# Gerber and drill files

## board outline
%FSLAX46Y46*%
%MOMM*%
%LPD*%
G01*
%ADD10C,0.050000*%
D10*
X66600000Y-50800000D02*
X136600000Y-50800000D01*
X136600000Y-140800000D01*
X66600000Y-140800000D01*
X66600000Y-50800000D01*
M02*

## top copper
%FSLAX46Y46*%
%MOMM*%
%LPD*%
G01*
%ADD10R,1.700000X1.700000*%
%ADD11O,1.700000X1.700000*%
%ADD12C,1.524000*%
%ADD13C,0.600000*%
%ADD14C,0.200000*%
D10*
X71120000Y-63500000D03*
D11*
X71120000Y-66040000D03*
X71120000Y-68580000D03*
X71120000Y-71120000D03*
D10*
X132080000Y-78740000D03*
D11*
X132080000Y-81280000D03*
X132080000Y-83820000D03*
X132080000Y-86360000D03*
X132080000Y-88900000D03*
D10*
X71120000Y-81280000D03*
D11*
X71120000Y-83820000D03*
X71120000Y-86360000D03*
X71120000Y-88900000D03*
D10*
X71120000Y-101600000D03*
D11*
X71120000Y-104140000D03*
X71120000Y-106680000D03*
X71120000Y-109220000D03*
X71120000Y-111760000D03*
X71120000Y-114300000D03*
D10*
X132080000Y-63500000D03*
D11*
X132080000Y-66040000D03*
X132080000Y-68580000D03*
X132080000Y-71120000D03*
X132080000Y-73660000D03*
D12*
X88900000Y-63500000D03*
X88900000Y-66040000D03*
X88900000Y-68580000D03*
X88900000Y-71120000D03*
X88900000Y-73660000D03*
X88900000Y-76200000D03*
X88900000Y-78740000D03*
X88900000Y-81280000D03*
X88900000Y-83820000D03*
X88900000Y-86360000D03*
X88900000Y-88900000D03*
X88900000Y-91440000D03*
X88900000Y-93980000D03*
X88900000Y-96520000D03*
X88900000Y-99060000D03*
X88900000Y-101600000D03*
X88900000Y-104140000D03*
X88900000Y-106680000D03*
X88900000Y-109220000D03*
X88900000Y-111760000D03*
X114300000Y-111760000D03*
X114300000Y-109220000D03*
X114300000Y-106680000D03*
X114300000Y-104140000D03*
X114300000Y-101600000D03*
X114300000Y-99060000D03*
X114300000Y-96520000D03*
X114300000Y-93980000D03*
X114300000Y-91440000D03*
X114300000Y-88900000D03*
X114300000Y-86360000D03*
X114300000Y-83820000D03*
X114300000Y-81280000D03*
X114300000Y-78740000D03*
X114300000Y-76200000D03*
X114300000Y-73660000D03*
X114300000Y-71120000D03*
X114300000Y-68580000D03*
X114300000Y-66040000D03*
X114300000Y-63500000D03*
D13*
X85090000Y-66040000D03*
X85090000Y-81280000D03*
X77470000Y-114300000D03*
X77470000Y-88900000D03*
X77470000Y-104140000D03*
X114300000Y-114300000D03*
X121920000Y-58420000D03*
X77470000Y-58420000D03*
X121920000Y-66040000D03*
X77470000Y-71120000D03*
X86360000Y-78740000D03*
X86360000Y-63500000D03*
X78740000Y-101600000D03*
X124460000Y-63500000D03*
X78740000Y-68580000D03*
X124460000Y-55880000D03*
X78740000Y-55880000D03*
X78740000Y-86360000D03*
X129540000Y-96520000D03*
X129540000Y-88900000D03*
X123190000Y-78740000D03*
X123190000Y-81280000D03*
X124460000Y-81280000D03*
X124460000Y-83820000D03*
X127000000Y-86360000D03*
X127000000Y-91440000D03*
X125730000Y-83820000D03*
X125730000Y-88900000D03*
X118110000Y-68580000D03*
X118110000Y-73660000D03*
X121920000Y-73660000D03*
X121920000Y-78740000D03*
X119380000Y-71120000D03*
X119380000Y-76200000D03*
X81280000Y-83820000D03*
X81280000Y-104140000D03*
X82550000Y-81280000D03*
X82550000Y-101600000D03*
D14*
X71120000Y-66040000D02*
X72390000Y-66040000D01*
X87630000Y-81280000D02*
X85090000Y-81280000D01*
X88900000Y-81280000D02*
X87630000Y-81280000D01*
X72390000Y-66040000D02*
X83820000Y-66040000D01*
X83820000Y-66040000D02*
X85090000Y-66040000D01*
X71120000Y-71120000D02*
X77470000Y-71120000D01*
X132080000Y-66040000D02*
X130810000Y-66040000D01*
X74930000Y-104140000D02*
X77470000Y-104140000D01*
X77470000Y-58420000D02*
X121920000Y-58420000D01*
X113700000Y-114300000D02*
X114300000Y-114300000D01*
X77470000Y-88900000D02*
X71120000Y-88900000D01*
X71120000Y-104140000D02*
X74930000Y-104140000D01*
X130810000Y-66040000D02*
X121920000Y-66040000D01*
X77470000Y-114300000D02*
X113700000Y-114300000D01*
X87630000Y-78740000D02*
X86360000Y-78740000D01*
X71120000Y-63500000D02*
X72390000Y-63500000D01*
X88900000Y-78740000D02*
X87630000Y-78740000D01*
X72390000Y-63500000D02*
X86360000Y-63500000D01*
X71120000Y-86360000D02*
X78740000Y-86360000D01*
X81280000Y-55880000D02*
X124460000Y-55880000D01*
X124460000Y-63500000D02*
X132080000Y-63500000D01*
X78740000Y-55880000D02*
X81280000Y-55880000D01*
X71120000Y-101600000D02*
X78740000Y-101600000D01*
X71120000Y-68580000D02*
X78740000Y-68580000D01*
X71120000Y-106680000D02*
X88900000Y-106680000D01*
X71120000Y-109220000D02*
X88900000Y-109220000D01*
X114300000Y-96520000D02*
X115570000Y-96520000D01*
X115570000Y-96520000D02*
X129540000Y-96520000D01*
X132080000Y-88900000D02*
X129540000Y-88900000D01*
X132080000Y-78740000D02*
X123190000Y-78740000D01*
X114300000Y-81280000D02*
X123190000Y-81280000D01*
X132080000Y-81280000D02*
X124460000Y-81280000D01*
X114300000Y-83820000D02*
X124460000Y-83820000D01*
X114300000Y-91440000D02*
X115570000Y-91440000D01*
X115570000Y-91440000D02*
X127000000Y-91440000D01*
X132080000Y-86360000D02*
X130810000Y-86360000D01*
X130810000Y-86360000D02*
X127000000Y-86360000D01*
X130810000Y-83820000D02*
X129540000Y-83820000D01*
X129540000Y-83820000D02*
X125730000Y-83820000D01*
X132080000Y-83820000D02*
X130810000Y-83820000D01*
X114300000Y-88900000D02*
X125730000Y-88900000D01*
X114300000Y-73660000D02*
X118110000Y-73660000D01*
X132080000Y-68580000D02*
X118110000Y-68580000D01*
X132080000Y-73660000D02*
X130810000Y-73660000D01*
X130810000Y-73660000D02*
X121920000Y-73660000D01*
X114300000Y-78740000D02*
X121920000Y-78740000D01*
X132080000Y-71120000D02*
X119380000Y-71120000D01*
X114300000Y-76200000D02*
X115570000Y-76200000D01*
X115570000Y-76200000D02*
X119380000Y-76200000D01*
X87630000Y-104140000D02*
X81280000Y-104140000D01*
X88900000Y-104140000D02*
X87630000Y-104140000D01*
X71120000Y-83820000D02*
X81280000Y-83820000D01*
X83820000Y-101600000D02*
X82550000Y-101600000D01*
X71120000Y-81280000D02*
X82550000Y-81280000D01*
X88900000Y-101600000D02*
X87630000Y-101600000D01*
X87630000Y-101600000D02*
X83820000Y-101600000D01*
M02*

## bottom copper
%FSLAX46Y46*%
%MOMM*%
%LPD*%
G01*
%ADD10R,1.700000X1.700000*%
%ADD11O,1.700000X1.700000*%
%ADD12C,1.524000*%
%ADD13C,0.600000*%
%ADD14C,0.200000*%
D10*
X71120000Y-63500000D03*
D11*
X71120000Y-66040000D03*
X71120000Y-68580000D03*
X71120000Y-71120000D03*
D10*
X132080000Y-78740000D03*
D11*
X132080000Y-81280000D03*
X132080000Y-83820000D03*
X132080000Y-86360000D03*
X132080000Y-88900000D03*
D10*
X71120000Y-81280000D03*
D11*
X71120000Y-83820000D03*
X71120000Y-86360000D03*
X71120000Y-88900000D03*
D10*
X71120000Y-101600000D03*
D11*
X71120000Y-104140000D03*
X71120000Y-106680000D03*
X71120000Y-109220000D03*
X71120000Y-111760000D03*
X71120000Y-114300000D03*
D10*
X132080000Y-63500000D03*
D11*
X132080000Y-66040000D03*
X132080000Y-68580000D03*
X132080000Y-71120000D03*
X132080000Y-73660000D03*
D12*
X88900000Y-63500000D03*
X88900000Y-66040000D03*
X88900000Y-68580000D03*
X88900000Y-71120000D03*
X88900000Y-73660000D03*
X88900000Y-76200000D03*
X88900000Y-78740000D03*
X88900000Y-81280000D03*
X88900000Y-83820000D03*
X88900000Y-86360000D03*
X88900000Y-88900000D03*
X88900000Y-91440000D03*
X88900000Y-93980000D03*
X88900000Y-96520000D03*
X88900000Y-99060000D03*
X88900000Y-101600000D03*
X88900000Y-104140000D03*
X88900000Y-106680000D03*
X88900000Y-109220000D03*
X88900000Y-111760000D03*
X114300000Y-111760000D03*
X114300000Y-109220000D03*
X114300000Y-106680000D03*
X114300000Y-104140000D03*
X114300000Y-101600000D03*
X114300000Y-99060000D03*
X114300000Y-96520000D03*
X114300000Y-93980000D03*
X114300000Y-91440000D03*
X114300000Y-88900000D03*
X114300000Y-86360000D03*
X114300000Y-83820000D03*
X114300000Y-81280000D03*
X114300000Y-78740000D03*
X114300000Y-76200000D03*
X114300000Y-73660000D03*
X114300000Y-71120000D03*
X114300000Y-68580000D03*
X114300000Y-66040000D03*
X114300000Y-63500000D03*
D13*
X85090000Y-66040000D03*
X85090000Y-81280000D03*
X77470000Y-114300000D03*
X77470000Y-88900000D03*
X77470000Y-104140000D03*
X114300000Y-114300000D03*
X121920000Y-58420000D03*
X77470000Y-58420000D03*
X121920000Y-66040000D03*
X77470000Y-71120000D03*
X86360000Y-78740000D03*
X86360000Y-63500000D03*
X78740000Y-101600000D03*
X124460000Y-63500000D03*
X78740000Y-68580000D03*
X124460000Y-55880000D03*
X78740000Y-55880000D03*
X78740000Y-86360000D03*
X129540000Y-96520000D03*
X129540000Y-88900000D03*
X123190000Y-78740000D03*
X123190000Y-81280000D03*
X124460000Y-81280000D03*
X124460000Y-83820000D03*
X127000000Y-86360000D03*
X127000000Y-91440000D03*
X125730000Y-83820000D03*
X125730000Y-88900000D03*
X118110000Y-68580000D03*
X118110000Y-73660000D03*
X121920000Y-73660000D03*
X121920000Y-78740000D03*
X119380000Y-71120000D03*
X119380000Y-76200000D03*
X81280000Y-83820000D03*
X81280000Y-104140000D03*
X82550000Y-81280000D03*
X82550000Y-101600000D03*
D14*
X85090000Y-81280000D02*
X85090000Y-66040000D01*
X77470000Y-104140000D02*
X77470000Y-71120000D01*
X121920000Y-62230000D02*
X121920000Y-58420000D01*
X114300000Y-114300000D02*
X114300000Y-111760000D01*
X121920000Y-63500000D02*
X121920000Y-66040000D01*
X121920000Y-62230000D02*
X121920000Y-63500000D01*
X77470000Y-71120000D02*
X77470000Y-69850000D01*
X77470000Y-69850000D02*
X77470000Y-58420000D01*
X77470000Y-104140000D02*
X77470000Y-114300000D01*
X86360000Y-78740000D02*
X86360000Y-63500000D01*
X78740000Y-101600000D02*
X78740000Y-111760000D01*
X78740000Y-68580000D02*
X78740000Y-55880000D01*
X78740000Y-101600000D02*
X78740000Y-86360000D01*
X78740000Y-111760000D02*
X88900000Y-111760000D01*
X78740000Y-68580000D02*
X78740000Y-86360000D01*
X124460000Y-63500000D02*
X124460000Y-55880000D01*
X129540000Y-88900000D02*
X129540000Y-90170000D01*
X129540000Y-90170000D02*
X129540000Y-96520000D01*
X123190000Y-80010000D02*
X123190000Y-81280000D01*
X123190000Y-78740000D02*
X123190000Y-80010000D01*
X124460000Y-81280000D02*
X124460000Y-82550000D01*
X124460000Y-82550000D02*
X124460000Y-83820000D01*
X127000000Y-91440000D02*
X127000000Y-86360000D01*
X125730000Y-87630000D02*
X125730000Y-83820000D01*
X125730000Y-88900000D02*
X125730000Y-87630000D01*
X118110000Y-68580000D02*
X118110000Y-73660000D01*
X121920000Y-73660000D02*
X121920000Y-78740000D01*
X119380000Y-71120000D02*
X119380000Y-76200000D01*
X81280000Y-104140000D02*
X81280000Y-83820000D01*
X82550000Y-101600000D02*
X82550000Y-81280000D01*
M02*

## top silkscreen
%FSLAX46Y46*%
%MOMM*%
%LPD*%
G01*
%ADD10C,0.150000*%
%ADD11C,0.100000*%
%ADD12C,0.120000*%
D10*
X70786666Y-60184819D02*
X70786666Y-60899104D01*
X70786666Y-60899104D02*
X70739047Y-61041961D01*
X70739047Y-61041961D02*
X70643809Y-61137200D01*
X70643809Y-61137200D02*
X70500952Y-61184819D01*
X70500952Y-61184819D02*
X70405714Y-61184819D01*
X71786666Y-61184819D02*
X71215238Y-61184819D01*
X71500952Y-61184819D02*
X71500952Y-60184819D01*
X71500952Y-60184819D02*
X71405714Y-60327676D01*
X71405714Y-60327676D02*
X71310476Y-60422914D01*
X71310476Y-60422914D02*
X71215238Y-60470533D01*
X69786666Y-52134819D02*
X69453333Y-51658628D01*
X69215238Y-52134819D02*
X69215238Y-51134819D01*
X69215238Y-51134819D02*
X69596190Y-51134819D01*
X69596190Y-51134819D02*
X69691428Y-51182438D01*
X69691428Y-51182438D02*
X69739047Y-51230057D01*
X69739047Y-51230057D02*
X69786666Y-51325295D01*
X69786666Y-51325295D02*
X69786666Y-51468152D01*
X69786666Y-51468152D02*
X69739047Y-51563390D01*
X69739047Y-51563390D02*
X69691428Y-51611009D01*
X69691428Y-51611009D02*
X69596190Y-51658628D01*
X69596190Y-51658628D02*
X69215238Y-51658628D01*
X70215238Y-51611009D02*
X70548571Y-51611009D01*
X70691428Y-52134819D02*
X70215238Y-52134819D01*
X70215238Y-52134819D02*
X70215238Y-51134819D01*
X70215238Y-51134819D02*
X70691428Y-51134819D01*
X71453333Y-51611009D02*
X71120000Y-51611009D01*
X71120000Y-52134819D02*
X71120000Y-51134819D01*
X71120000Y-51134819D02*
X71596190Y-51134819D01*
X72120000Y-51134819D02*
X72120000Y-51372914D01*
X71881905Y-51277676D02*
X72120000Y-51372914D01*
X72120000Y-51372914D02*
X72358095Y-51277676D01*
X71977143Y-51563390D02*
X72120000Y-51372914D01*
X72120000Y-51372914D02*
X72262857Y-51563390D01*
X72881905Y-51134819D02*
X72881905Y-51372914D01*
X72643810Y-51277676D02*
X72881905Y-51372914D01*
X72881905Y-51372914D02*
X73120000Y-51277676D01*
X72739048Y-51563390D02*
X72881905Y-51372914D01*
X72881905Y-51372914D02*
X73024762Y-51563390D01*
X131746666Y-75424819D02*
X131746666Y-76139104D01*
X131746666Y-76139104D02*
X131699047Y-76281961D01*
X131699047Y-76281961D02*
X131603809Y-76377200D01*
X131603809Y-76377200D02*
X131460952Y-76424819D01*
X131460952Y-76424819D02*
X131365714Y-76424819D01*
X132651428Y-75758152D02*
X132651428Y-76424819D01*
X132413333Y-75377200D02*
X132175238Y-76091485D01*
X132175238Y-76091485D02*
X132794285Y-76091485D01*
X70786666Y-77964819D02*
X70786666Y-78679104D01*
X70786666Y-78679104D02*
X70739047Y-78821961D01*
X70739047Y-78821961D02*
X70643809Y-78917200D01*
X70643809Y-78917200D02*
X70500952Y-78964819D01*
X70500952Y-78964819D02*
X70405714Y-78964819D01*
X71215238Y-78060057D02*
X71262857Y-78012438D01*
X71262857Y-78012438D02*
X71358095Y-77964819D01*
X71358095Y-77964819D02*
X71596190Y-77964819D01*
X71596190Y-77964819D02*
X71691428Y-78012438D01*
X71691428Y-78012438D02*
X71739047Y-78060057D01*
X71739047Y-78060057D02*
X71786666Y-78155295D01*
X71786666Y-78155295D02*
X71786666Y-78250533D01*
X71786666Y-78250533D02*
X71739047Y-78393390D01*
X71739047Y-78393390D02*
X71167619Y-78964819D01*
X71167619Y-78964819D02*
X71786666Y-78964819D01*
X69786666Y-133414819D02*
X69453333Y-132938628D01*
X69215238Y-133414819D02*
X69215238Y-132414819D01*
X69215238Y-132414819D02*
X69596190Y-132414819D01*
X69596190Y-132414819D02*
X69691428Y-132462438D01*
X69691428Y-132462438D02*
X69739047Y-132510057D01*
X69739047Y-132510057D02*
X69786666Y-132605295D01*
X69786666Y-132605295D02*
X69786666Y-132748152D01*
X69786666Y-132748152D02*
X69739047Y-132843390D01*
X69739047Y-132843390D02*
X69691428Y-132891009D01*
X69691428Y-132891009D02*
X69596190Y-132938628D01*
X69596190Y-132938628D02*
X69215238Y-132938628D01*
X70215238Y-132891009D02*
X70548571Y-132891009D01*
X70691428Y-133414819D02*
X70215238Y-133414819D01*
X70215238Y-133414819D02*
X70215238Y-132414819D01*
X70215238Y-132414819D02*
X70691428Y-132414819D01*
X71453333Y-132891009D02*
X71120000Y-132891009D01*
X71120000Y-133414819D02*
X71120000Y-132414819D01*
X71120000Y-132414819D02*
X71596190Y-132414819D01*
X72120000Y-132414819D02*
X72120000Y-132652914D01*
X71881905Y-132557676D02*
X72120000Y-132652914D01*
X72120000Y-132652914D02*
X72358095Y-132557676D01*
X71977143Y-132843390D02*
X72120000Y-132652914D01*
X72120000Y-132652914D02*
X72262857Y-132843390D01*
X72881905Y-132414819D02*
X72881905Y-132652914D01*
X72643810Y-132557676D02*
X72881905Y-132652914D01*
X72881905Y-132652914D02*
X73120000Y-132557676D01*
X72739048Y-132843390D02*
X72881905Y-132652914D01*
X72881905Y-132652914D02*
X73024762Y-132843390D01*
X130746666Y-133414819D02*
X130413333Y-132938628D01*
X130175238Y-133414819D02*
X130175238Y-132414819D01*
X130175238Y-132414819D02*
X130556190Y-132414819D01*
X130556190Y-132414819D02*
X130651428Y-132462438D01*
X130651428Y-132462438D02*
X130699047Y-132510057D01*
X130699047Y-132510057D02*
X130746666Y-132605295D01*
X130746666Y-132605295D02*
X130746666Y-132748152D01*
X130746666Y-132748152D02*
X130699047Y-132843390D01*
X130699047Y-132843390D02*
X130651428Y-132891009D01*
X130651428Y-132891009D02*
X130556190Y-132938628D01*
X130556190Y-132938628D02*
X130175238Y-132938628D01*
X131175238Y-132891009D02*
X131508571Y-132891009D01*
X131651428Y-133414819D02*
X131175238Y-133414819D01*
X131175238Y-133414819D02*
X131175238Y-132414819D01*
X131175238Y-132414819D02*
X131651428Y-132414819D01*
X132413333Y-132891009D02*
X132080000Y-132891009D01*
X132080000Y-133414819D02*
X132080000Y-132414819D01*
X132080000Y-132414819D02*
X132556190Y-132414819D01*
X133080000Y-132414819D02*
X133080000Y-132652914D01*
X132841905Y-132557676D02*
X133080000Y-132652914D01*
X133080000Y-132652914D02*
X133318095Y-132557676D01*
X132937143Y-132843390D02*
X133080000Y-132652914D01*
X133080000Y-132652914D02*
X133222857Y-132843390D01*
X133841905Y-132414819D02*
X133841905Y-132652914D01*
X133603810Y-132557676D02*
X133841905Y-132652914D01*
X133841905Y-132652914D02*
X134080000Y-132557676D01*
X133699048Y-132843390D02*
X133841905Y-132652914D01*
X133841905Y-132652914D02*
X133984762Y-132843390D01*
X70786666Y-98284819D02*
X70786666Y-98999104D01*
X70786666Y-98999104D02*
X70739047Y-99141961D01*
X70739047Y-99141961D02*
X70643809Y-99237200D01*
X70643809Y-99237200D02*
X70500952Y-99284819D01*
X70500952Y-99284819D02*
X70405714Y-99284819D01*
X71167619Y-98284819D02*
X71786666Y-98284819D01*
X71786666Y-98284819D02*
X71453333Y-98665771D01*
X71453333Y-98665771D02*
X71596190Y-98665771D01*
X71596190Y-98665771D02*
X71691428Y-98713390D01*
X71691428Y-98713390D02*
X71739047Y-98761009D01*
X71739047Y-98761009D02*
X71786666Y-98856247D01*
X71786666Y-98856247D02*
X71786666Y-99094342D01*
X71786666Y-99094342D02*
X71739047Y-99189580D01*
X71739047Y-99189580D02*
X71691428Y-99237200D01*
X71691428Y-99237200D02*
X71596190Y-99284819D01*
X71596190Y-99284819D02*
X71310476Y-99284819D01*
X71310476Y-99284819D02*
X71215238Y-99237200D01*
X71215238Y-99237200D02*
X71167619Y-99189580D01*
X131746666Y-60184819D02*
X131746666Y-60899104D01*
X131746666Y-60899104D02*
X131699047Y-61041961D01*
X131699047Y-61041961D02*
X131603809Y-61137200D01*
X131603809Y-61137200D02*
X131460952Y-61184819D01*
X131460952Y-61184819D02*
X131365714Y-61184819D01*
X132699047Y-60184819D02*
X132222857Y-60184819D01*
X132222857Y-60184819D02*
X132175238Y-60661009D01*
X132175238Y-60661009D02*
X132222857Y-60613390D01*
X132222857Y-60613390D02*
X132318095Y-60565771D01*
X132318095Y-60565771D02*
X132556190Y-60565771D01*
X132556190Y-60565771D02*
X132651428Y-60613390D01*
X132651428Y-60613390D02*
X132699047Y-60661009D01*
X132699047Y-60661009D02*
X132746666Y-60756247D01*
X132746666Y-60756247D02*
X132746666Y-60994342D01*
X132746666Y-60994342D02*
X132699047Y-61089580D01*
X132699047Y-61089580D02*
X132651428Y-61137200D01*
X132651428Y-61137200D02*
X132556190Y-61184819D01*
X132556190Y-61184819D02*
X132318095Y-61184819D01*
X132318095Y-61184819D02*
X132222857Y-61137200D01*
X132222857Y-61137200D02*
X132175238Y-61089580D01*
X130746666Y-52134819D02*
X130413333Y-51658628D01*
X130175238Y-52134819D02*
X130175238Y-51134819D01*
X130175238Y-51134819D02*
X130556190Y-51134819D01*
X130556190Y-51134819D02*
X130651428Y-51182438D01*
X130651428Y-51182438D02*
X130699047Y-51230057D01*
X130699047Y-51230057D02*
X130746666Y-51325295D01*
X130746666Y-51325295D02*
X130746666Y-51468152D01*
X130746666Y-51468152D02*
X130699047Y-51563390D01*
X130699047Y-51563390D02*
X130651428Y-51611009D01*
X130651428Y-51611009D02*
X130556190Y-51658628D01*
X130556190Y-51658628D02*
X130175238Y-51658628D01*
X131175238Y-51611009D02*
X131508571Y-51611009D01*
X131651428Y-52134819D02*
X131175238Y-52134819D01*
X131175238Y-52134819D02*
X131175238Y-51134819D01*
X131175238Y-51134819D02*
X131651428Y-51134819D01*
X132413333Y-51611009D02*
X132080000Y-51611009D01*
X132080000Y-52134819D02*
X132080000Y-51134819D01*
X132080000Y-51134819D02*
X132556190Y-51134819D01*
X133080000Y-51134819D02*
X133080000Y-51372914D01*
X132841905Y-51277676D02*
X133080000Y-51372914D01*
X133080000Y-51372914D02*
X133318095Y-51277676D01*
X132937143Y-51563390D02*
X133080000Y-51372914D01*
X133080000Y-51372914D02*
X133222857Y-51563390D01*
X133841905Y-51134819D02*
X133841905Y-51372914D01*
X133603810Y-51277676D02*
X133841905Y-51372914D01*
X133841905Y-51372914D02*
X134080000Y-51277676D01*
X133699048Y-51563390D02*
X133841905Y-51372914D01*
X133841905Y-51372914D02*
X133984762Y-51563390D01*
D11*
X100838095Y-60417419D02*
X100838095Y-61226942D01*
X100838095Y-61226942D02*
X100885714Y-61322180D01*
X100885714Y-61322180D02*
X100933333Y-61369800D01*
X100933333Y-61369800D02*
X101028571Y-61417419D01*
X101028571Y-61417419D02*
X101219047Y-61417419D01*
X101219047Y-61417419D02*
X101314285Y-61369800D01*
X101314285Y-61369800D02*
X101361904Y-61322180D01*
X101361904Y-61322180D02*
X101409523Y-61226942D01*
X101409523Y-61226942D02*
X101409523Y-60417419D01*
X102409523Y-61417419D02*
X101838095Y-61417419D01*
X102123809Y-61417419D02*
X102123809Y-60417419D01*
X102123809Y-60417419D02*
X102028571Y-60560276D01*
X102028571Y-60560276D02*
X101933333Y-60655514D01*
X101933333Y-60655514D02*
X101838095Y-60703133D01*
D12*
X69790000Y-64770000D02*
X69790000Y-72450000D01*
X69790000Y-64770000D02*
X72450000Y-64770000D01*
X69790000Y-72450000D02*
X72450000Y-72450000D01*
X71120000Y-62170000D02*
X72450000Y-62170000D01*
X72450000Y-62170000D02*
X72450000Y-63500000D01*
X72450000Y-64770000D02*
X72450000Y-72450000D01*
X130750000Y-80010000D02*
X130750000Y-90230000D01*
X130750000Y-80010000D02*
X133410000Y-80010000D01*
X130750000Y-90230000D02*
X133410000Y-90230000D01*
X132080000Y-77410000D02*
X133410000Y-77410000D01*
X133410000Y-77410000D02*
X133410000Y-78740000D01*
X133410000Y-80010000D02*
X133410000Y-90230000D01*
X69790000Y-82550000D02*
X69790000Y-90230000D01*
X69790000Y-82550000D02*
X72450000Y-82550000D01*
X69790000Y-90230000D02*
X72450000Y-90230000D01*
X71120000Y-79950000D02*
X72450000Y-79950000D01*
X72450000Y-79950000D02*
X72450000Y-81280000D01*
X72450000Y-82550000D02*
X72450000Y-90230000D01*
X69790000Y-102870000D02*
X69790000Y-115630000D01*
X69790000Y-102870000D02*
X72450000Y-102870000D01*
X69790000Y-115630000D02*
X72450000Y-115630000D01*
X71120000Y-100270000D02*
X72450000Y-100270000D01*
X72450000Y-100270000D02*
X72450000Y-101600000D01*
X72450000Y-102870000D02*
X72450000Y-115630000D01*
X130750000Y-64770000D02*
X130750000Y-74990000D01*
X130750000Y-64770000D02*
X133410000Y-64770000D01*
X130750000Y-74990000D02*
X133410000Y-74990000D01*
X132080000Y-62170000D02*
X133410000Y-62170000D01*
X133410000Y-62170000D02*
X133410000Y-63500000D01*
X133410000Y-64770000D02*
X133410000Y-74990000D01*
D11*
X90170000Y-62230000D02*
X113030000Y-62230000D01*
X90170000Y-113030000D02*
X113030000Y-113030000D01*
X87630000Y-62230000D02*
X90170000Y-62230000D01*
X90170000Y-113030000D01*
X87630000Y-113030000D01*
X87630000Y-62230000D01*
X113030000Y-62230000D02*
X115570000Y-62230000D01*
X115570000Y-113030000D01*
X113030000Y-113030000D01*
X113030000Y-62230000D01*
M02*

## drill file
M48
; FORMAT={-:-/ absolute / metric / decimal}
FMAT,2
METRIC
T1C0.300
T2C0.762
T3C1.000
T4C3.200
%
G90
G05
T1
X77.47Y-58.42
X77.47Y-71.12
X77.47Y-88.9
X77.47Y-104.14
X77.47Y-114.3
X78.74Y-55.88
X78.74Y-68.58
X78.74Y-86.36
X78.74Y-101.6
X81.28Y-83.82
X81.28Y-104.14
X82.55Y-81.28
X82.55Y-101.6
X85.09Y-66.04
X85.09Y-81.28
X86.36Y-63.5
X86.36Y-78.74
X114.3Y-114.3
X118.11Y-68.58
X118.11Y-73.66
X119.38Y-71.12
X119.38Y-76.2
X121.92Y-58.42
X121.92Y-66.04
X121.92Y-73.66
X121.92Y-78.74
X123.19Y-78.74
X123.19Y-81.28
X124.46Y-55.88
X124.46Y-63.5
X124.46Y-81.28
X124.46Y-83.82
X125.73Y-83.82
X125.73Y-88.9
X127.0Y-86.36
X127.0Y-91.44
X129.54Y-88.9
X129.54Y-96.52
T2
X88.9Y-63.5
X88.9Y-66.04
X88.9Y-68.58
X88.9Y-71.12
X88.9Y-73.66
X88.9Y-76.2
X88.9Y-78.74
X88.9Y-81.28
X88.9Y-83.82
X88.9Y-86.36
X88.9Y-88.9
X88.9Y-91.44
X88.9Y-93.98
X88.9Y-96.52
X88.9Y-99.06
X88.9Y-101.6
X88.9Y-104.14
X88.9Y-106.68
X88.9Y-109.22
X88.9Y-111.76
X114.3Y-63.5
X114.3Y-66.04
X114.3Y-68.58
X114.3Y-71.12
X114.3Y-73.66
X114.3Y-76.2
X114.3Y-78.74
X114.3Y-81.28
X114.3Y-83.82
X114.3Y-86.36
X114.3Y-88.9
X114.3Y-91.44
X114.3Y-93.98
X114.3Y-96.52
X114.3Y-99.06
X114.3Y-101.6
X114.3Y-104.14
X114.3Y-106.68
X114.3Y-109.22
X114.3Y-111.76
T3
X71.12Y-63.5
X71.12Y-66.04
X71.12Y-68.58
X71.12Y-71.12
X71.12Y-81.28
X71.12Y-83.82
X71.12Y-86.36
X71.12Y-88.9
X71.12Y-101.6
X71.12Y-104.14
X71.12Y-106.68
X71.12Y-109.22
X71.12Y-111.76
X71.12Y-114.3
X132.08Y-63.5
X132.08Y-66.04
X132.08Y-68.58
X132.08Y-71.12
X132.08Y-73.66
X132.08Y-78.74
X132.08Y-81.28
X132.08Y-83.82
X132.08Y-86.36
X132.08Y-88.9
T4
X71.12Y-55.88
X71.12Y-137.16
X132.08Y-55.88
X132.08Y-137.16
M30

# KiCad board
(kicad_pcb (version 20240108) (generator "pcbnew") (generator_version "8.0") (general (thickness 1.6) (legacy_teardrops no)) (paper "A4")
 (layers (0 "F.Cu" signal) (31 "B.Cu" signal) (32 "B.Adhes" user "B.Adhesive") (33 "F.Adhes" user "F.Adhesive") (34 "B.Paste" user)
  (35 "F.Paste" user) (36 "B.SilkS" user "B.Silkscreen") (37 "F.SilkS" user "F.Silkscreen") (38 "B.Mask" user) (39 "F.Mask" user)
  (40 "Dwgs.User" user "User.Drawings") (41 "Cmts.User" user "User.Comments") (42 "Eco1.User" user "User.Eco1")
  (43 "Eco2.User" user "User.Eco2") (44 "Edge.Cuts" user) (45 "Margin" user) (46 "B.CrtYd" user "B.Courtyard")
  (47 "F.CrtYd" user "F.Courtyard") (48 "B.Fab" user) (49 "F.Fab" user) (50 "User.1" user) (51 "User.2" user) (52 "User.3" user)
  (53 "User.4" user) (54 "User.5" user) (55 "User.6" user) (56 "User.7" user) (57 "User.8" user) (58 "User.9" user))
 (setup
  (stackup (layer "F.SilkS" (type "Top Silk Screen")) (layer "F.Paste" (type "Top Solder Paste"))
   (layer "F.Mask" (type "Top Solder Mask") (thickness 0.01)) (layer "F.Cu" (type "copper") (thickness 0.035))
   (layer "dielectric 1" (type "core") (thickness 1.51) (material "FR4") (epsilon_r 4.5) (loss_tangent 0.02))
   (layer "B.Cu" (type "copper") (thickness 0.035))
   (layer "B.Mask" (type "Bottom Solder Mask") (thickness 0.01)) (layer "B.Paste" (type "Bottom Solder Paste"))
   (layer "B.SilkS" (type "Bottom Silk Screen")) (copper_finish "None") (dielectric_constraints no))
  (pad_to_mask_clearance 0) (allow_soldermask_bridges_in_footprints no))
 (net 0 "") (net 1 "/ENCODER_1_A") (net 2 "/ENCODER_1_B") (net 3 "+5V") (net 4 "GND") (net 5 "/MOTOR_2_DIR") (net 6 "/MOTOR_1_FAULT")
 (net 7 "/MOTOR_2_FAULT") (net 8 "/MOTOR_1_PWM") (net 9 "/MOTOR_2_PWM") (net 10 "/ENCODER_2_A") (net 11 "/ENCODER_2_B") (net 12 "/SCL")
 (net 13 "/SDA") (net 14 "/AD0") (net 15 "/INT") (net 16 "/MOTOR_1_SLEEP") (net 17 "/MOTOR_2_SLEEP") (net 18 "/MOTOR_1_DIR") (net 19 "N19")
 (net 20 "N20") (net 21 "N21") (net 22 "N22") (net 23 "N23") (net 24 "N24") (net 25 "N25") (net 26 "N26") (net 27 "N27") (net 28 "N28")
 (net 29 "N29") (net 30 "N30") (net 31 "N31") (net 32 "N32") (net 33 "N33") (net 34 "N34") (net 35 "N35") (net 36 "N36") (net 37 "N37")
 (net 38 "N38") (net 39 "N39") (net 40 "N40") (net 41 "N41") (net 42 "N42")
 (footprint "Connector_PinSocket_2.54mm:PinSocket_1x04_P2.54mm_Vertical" (layer "F.Cu") (at 71.12 63.5)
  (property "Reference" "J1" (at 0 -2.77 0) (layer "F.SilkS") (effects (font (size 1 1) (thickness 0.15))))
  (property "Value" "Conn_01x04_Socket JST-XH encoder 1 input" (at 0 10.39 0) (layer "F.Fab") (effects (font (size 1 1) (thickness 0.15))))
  (fp_line (start -1.33 1.27) (end -1.33 8.95) (stroke (width 0.12) (type solid)) (layer "F.SilkS"))
  (fp_line (start -1.33 1.27) (end 1.33 1.27) (stroke (width 0.12) (type solid)) (layer "F.SilkS"))
  (fp_line (start -1.33 8.95) (end 1.33 8.95) (stroke (width 0.12) (type solid)) (layer "F.SilkS"))
  (fp_line (start 0 -1.33) (end 1.33 -1.33) (stroke (width 0.12) (type solid)) (layer "F.SilkS"))
  (fp_line (start 1.33 -1.33) (end 1.33 0) (stroke (width 0.12) (type solid)) (layer "F.SilkS"))
  (fp_line (start 1.33 1.27) (end 1.33 8.95) (stroke (width 0.12) (type solid)) (layer "F.SilkS"))
  (pad "1" thru_hole rect (at 0 0) (size 1.7 1.7) (drill 1) (layers "*.Cu" "*.Mask") (remove_unused_layers no) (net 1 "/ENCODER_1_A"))
  (pad "2" thru_hole oval (at 0 2.54) (size 1.7 1.7) (drill 1) (layers "*.Cu" "*.Mask") (remove_unused_layers no) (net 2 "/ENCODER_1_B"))
  (pad "3" thru_hole oval (at 0 5.08) (size 1.7 1.7) (drill 1) (layers "*.Cu" "*.Mask") (remove_unused_layers no) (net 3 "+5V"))
  (pad "4" thru_hole oval (at 0 7.62) (size 1.7 1.7) (drill 1) (layers "*.Cu" "*.Mask") (remove_unused_layers no) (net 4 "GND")))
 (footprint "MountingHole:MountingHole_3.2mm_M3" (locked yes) (layer "F.Cu") (at 71.12 55.88)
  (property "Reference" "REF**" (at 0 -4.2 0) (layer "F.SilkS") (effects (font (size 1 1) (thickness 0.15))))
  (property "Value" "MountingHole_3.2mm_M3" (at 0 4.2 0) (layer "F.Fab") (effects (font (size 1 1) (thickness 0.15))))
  (pad "" np_thru_hole circle (at 0 0) (size 3.2 3.2) (drill 3.2) (layers "*.Cu" "*.Mask")))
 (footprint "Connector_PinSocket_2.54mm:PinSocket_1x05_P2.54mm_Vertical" (layer "F.Cu") (at 132.08 78.74)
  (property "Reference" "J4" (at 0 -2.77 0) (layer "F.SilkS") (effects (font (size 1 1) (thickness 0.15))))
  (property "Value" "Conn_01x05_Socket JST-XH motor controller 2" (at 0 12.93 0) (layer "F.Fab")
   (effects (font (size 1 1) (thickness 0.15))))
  (fp_line (start -1.33 1.27) (end -1.33 11.49) (stroke (width 0.12) (type solid)) (layer "F.SilkS"))
  (fp_line (start -1.33 1.27) (end 1.33 1.27) (stroke (width 0.12) (type solid)) (layer "F.SilkS"))
  (fp_line (start -1.33 11.49) (end 1.33 11.49) (stroke (width 0.12) (type solid)) (layer "F.SilkS"))
  (fp_line (start 0 -1.33) (end 1.33 -1.33) (stroke (width 0.12) (type solid)) (layer "F.SilkS"))
  (fp_line (start 1.33 -1.33) (end 1.33 0) (stroke (width 0.12) (type solid)) (layer "F.SilkS"))
  (fp_line (start 1.33 1.27) (end 1.33 11.49) (stroke (width 0.12) (type solid)) (layer "F.SilkS"))
  (pad "1" thru_hole rect (at 0 0) (size 1.7 1.7) (drill 1) (layers "*.Cu" "*.Mask") (remove_unused_layers no) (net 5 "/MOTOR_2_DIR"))
  (pad "2" thru_hole oval (at 0 2.54) (size 1.7 1.7) (drill 1) (layers "*.Cu" "*.Mask") (remove_unused_layers no) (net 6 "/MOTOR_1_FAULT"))
  (pad "3" thru_hole oval (at 0 5.08) (size 1.7 1.7) (drill 1) (layers "*.Cu" "*.Mask") (remove_unused_layers no) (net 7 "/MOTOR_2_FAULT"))
  (pad "4" thru_hole oval (at 0 7.62) (size 1.7 1.7) (drill 1) (layers "*.Cu" "*.Mask") (remove_unused_layers no) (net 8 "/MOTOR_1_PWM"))
  (pad "5" thru_hole oval (at 0 10.16) (size 1.7 1.7) (drill 1) (layers "*.Cu" "*.Mask") (remove_unused_layers no) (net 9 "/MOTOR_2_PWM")))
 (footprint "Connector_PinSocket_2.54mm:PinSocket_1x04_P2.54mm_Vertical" (layer "F.Cu") (at 71.12 81.28)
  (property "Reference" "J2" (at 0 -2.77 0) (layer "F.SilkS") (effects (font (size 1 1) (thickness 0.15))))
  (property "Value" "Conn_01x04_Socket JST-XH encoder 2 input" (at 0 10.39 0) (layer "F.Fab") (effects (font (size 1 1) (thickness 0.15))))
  (fp_line (start -1.33 1.27) (end -1.33 8.95) (stroke (width 0.12) (type solid)) (layer "F.SilkS"))
  (fp_line (start -1.33 1.27) (end 1.33 1.27) (stroke (width 0.12) (type solid)) (layer "F.SilkS"))
  (fp_line (start -1.33 8.95) (end 1.33 8.95) (stroke (width 0.12) (type solid)) (layer "F.SilkS"))
  (fp_line (start 0 -1.33) (end 1.33 -1.33) (stroke (width 0.12) (type solid)) (layer "F.SilkS"))
  (fp_line (start 1.33 -1.33) (end 1.33 0) (stroke (width 0.12) (type solid)) (layer "F.SilkS"))
  (fp_line (start 1.33 1.27) (end 1.33 8.95) (stroke (width 0.12) (type solid)) (layer "F.SilkS"))
  (pad "1" thru_hole rect (at 0 0) (size 1.7 1.7) (drill 1) (layers "*.Cu" "*.Mask") (remove_unused_layers no) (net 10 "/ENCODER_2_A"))
  (pad "2" thru_hole oval (at 0 2.54) (size 1.7 1.7) (drill 1) (layers "*.Cu" "*.Mask") (remove_unused_layers no) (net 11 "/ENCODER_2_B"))
  (pad "3" thru_hole oval (at 0 5.08) (size 1.7 1.7) (drill 1) (layers "*.Cu" "*.Mask") (remove_unused_layers no) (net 3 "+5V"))
  (pad "4" thru_hole oval (at 0 7.62) (size 1.7 1.7) (drill 1) (layers "*.Cu" "*.Mask") (remove_unused_layers no) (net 4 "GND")))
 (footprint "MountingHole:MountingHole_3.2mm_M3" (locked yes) (layer "F.Cu") (at 71.12 137.16)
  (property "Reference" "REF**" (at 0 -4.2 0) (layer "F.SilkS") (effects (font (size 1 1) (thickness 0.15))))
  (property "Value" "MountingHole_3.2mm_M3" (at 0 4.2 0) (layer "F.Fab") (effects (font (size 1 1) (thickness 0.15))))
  (pad "" np_thru_hole circle (at 0 0) (size 3.2 3.2) (drill 3.2) (layers "*.Cu" "*.Mask")))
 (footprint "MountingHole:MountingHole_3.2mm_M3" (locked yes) (layer "F.Cu") (at 132.08 137.16)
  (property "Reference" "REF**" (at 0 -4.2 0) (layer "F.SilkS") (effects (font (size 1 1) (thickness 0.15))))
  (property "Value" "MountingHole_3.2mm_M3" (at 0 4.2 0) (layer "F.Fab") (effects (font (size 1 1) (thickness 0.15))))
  (pad "" np_thru_hole circle (at 0 0) (size 3.2 3.2) (drill 3.2) (layers "*.Cu" "*.Mask")))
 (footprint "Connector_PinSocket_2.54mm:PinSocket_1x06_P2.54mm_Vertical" (layer "F.Cu") (at 71.12 101.6)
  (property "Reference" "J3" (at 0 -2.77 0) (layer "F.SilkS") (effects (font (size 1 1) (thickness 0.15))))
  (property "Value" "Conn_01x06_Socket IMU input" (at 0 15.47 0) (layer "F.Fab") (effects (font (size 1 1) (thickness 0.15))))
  (fp_line (start -1.33 1.27) (end -1.33 14.03) (stroke (width 0.12) (type solid)) (layer "F.SilkS"))
  (fp_line (start -1.33 1.27) (end 1.33 1.27) (stroke (width 0.12) (type solid)) (layer "F.SilkS"))
  (fp_line (start -1.33 14.03) (end 1.33 14.03) (stroke (width 0.12) (type solid)) (layer "F.SilkS"))
  (fp_line (start 0 -1.33) (end 1.33 -1.33) (stroke (width 0.12) (type solid)) (layer "F.SilkS"))
  (fp_line (start 1.33 -1.33) (end 1.33 0) (stroke (width 0.12) (type solid)) (layer "F.SilkS"))
  (fp_line (start 1.33 1.27) (end 1.33 14.03) (stroke (width 0.12) (type solid)) (layer "F.SilkS"))
  (pad "1" thru_hole rect (at 0 0) (size 1.7 1.7) (drill 1) (layers "*.Cu" "*.Mask") (remove_unused_layers no) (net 3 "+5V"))
  (pad "2" thru_hole oval (at 0 2.54) (size 1.7 1.7) (drill 1) (layers "*.Cu" "*.Mask") (remove_unused_layers no) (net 4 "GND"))
  (pad "3" thru_hole oval (at 0 5.08) (size 1.7 1.7) (drill 1) (layers "*.Cu" "*.Mask") (remove_unused_layers no) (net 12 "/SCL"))
  (pad "4" thru_hole oval (at 0 7.62) (size 1.7 1.7) (drill 1) (layers "*.Cu" "*.Mask") (remove_unused_layers no) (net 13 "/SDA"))
  (pad "5" thru_hole oval (at 0 10.16) (size 1.7 1.7) (drill 1) (layers "*.Cu" "*.Mask") (remove_unused_layers no) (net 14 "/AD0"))
  (pad "6" thru_hole oval (at 0 12.7) (size 1.7 1.7) (drill 1) (layers "*.Cu" "*.Mask") (remove_unused_layers no) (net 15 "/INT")))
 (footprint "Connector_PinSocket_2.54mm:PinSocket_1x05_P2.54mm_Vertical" (layer "F.Cu") (at 132.08 63.5)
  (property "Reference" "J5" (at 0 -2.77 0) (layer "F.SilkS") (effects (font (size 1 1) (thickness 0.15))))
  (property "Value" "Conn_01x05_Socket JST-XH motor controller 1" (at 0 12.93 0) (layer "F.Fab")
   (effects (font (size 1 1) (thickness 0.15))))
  (fp_line (start -1.33 1.27) (end -1.33 11.49) (stroke (width 0.12) (type solid)) (layer "F.SilkS"))
  (fp_line (start -1.33 1.27) (end 1.33 1.27) (stroke (width 0.12) (type solid)) (layer "F.SilkS"))
  (fp_line (start -1.33 11.49) (end 1.33 11.49) (stroke (width 0.12) (type solid)) (layer "F.SilkS"))
  (fp_line (start 0 -1.33) (end 1.33 -1.33) (stroke (width 0.12) (type solid)) (layer "F.SilkS"))
  (fp_line (start 1.33 -1.33) (end 1.33 0) (stroke (width 0.12) (type solid)) (layer "F.SilkS"))
  (fp_line (start 1.33 1.27) (end 1.33 11.49) (stroke (width 0.12) (type solid)) (layer "F.SilkS"))
  (pad "1" thru_hole rect (at 0 0) (size 1.7 1.7) (drill 1) (layers "*.Cu" "*.Mask") (remove_unused_layers no) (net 3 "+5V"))
  (pad "2" thru_hole oval (at 0 2.54) (size 1.7 1.7) (drill 1) (layers "*.Cu" "*.Mask") (remove_unused_layers no) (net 4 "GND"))
  (pad "3" thru_hole oval (at 0 5.08) (size 1.7 1.7) (drill 1) (layers "*.Cu" "*.Mask") (remove_unused_layers no) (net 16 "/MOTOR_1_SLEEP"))
  (pad "4" thru_hole oval (at 0 7.62) (size 1.7 1.7) (drill 1) (layers "*.Cu" "*.Mask") (remove_unused_layers no) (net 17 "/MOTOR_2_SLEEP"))
  (pad "5" thru_hole oval (at 0 10.16) (size 1.7 1.7) (drill 1) (layers "*.Cu" "*.Mask") (remove_unused_layers no) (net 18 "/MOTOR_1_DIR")))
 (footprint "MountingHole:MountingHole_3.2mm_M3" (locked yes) (layer "F.Cu") (at 132.08 55.88)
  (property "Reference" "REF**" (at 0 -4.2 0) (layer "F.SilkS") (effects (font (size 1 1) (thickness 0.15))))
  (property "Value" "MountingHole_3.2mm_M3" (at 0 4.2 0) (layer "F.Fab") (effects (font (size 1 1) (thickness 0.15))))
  (pad "" np_thru_hole circle (at 0 0) (size 3.2 3.2) (drill 3.2) (layers "*.Cu" "*.Mask")))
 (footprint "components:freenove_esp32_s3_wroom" (layer "F.Cu") (at 88.9 63.5)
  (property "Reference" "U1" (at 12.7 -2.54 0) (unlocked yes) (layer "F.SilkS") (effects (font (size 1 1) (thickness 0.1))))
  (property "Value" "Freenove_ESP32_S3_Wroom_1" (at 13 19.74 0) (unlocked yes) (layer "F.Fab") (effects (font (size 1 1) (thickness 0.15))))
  (fp_line (start 1.27 -1.27) (end 24.13 -1.27) (stroke (width 0.1) (type default)) (layer "F.SilkS"))
  (fp_line (start 1.27 49.53) (end 24.13 49.53) (stroke (width 0.1) (type default)) (layer "F.SilkS"))
  (fp_rect (start -1.27 -1.27) (end 1.27 49.53) (stroke (width 0.1) (type default)) (fill none) (layer "F.SilkS"))
  (fp_rect (start 24.13 -1.27) (end 26.67 49.53) (stroke (width 0.1) (type default)) (fill none) (layer "F.SilkS"))
  (pad "1" thru_hole circle (at 0 0) (size 1.524 1.524) (drill 0.762) (layers "*.Cu" "*.Mask") (remove_unused_layers no) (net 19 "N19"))
  (pad "2" thru_hole circle (at 0 2.54) (size 1.524 1.524) (drill 0.762) (layers "*.Cu" "*.Mask") (remove_unused_layers no) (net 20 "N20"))
  (pad "3" thru_hole circle (at 0 5.08) (size 1.524 1.524) (drill 0.762) (layers "*.Cu" "*.Mask") (remove_unused_layers no) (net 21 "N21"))
  (pad "4" thru_hole circle (at 0 7.62) (size 1.524 1.524) (drill 0.762) (layers "*.Cu" "*.Mask") (remove_unused_layers no) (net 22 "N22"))
  (pad "5" thru_hole circle (at 0 10.16) (size 1.524 1.524) (drill 0.762) (layers "*.Cu" "*.Mask") (remove_unused_layers no) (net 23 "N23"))
  (pad "6" thru_hole circle (at 0 12.7) (size 1.524 1.524) (drill 0.762) (layers "*.Cu" "*.Mask") (remove_unused_layers no) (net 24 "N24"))
  (pad "7" thru_hole circle (at 0 15.24) (size 1.524 1.524) (drill 0.762) (layers "*.Cu" "*.Mask") (remove_unused_layers no)
   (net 1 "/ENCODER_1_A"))
  (pad "8" thru_hole circle (at 0 17.78) (size 1.524 1.524) (drill 0.762) (layers "*.Cu" "*.Mask") (remove_unused_layers no)
   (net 2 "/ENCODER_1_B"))
  (pad "9" thru_hole circle (at 0 20.32) (size 1.524 1.524) (drill 0.762) (layers "*.Cu" "*.Mask") (remove_unused_layers no) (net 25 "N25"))
  (pad "10" thru_hole circle (at 0 22.86) (size 1.524 1.524) (drill 0.762) (layers "*.Cu" "*.Mask") (remove_unused_layers no) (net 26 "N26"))
  (pad "11" thru_hole circle (at 0 25.4) (size 1.524 1.524) (drill 0.762) (layers "*.Cu" "*.Mask") (remove_unused_layers no) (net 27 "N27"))
  (pad "12" thru_hole circle (at 0 27.94) (size 1.524 1.524) (drill 0.762) (layers "*.Cu" "*.Mask") (remove_unused_layers no) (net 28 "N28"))
  (pad "13" thru_hole circle (at 0 30.48) (size 1.524 1.524) (drill 0.762) (layers "*.Cu" "*.Mask") (remove_unused_layers no) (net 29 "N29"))
  (pad "14" thru_hole circle (at 0 33.02) (size 1.524 1.524) (drill 0.762) (layers "*.Cu" "*.Mask") (remove_unused_layers no) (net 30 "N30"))
  (pad "15" thru_hole circle (at 0 35.56) (size 1.524 1.524) (drill 0.762) (layers "*.Cu" "*.Mask") (remove_unused_layers no) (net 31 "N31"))
  (pad "16" thru_hole circle (at 0 38.1) (size 1.524 1.524) (drill 0.762) (layers "*.Cu" "*.Mask") (remove_unused_layers no)
   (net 10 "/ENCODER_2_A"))
  (pad "17" thru_hole circle (at 0 40.64) (size 1.524 1.524) (drill 0.762) (layers "*.Cu" "*.Mask") (remove_unused_layers no)
   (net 11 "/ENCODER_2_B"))
  (pad "18" thru_hole circle (at 0 43.18) (size 1.524 1.524) (drill 0.762) (layers "*.Cu" "*.Mask") (remove_unused_layers no)
   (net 12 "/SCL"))
  (pad "19" thru_hole circle (at 0 45.72) (size 1.524 1.524) (drill 0.762) (layers "*.Cu" "*.Mask") (remove_unused_layers no)
   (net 13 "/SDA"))
  (pad "20" thru_hole circle (at 0 48.26) (size 1.524 1.524) (drill 0.762) (layers "*.Cu" "*.Mask") (remove_unused_layers no) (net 3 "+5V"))
  (pad "21" thru_hole circle (at 25.4 48.26) (size 1.524 1.524) (drill 0.762) (layers "*.Cu" "*.Mask") (remove_unused_layers no)
   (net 4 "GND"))
  (pad "22" thru_hole circle (at 25.4 45.72) (size 1.524 1.524) (drill 0.762) (layers "*.Cu" "*.Mask") (remove_unused_layers no)
   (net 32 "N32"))
  (pad "23" thru_hole circle (at 25.4 43.18) (size 1.524 1.524) (drill 0.762) (layers "*.Cu" "*.Mask") (remove_unused_layers no)
   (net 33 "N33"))
  (pad "24" thru_hole circle (at 25.4 40.64) (size 1.524 1.524) (drill 0.762) (layers "*.Cu" "*.Mask") (remove_unused_layers no)
   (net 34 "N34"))
  (pad "25" thru_hole circle (at 25.4 38.1) (size 1.524 1.524) (drill 0.762) (layers "*.Cu" "*.Mask") (remove_unused_layers no)
   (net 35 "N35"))
  (pad "26" thru_hole circle (at 25.4 35.56) (size 1.524 1.524) (drill 0.762) (layers "*.Cu" "*.Mask") (remove_unused_layers no)
   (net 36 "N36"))
  (pad "27" thru_hole circle (at 25.4 33.02) (size 1.524 1.524) (drill 0.762) (layers "*.Cu" "*.Mask") (remove_unused_layers no)
   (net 9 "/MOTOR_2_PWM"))
  (pad "28" thru_hole circle (at 25.4 30.48) (size 1.524 1.524) (drill 0.762) (layers "*.Cu" "*.Mask") (remove_unused_layers no)
   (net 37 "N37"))
  (pad "29" thru_hole circle (at 25.4 27.94) (size 1.524 1.524) (drill 0.762) (layers "*.Cu" "*.Mask") (remove_unused_layers no)
   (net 8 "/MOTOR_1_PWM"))
  (pad "30" thru_hole circle (at 25.4 25.4) (size 1.524 1.524) (drill 0.762) (layers "*.Cu" "*.Mask") (remove_unused_layers no)
   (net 7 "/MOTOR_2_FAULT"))
  (pad "31" thru_hole circle (at 25.4 22.86) (size 1.524 1.524) (drill 0.762) (layers "*.Cu" "*.Mask") (remove_unused_layers no)
   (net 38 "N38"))
  (pad "32" thru_hole circle (at 25.4 20.32) (size 1.524 1.524) (drill 0.762) (layers "*.Cu" "*.Mask") (remove_unused_layers no)
   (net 6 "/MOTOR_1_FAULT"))
  (pad "33" thru_hole circle (at 25.4 17.78) (size 1.524 1.524) (drill 0.762) (layers "*.Cu" "*.Mask") (remove_unused_layers no)
   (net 5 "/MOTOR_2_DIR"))
  (pad "34" thru_hole circle (at 25.4 15.24) (size 1.524 1.524) (drill 0.762) (layers "*.Cu" "*.Mask") (remove_unused_layers no)
   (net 18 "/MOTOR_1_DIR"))
  (pad "35" thru_hole circle (at 25.4 12.7) (size 1.524 1.524) (drill 0.762) (layers "*.Cu" "*.Mask") (remove_unused_layers no)
   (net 17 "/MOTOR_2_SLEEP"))
  (pad "36" thru_hole circle (at 25.4 10.16) (size 1.524 1.524) (drill 0.762) (layers "*.Cu" "*.Mask") (remove_unused_layers no)
   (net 16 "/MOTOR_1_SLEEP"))
  (pad "37" thru_hole circle (at 25.4 7.62) (size 1.524 1.524) (drill 0.762) (layers "*.Cu" "*.Mask") (remove_unused_layers no)
   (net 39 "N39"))
  (pad "38" thru_hole circle (at 25.4 5.08) (size 1.524 1.524) (drill 0.762) (layers "*.Cu" "*.Mask") (remove_unused_layers no)
   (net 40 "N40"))
  (pad "39" thru_hole circle (at 25.4 2.54) (size 1.524 1.524) (drill 0.762) (layers "*.Cu" "*.Mask") (remove_unused_layers no)
   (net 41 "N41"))
  (pad "40" thru_hole circle (at 25.4 0) (size 1.524 1.524) (drill 0.762) (layers "*.Cu" "*.Mask") (remove_unused_layers no) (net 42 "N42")))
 (gr_rect (start 66.6 50.8) (end 136.6 140.8) (locked yes) (stroke (width 0.05) (type default)) (fill none) (layer "Edge.Cuts"))
 (segment (start 71.12 66.04) (end 72.39 66.04) (width 0.2) (layer "F.Cu") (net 2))
 (segment (start 87.63 81.28) (end 85.09 81.28) (width 0.2) (layer "F.Cu") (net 2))
 (segment (start 88.9 81.28) (end 87.63 81.28) (width 0.2) (layer "F.Cu") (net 2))
 (segment (start 72.39 66.04) (end 83.82 66.04) (width 0.2) (layer "F.Cu") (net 2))
 (segment (start 83.82 66.04) (end 85.09 66.04) (width 0.2) (layer "F.Cu") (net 2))
 (via (at 85.09 66.04) (size 0.6) (drill 0.3) (layers "F.Cu" "B.Cu") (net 2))
 (via (at 85.09 81.28) (size 0.6) (drill 0.3) (layers "F.Cu" "B.Cu") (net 2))
 (segment (start 85.09 81.28) (end 85.09 66.04) (width 0.2) (layer "B.Cu") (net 2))
 (segment (start 71.12 71.12) (end 77.47 71.12) (width 0.2) (layer "F.Cu") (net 4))
 (segment (start 132.08 66.04) (end 130.81 66.04) (width 0.2) (layer "F.Cu") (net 4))
 (segment (start 74.93 104.14) (end 77.47 104.14) (width 0.2) (layer "F.Cu") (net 4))
 (segment (start 77.47 58.42) (end 121.92 58.42) (width 0.2) (layer "F.Cu") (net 4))
 (segment (start 113.7 114.3) (end 114.3 114.3) (width 0.2) (layer "F.Cu") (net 4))
 (segment (start 77.47 88.9) (end 71.12 88.9) (width 0.2) (layer "F.Cu") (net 4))
 (segment (start 71.12 104.14) (end 74.93 104.14) (width 0.2) (layer "F.Cu") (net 4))
 (segment (start 130.81 66.04) (end 121.92 66.04) (width 0.2) (layer "F.Cu") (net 4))
 (segment (start 77.47 114.3) (end 113.7 114.3) (width 0.2) (layer "F.Cu") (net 4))
 (via (at 77.47 114.3) (size 0.6) (drill 0.3) (layers "F.Cu" "B.Cu") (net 4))
 (via (at 77.47 88.9) (size 0.6) (drill 0.3) (layers "F.Cu" "B.Cu") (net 4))
 (via (at 77.47 104.14) (size 0.6) (drill 0.3) (layers "F.Cu" "B.Cu") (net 4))
 (via (at 114.3 114.3) (size 0.6) (drill 0.3) (layers "F.Cu" "B.Cu") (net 4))
 (via (at 121.92 58.42) (size 0.6) (drill 0.3) (layers "F.Cu" "B.Cu") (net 4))
 (via (at 77.47 58.42) (size 0.6) (drill 0.3) (layers "F.Cu" "B.Cu") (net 4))
 (via (at 121.92 66.04) (size 0.6) (drill 0.3) (layers "F.Cu" "B.Cu") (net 4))
 (via (at 77.47 71.12) (size 0.6) (drill 0.3) (layers "F.Cu" "B.Cu") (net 4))
 (segment (start 77.47 104.14) (end 77.47 71.12) (width 0.2) (layer "B.Cu") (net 4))
 (segment (start 121.92 62.23) (end 121.92 58.42) (width 0.2) (layer "B.Cu") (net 4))
 (segment (start 114.3 114.3) (end 114.3 111.76) (width 0.2) (layer "B.Cu") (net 4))
 (segment (start 121.92 63.5) (end 121.92 66.04) (width 0.2) (layer "B.Cu") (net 4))
 (segment (start 121.92 62.23) (end 121.92 63.5) (width 0.2) (layer "B.Cu") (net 4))
 (segment (start 77.47 71.12) (end 77.47 69.85) (width 0.2) (layer "B.Cu") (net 4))
 (segment (start 77.47 69.85) (end 77.47 58.42) (width 0.2) (layer "B.Cu") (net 4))
 (segment (start 77.47 104.14) (end 77.47 114.3) (width 0.2) (layer "B.Cu") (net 4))
 (segment (start 87.63 78.74) (end 86.36 78.74) (width 0.2) (layer "F.Cu") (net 1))
 (segment (start 71.12 63.5) (end 72.39 63.5) (width 0.2) (layer "F.Cu") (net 1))
 (segment (start 88.9 78.74) (end 87.63 78.74) (width 0.2) (layer "F.Cu") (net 1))
 (segment (start 72.39 63.5) (end 86.36 63.5) (width 0.2) (layer "F.Cu") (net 1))
 (via (at 86.36 78.74) (size 0.6) (drill 0.3) (layers "F.Cu" "B.Cu") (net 1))
 (via (at 86.36 63.5) (size 0.6) (drill 0.3) (layers "F.Cu" "B.Cu") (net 1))
 (segment (start 86.36 78.74) (end 86.36 63.5) (width 0.2) (layer "B.Cu") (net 1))
 (segment (start 71.12 86.36) (end 78.74 86.36) (width 0.2) (layer "F.Cu") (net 3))
 (segment (start 81.28 55.88) (end 124.46 55.88) (width 0.2) (layer "F.Cu") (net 3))
 (segment (start 124.46 63.5) (end 132.08 63.5) (width 0.2) (layer "F.Cu") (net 3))
 (segment (start 78.74 55.88) (end 81.28 55.88) (width 0.2) (layer "F.Cu") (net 3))
 (segment (start 71.12 101.6) (end 78.74 101.6) (width 0.2) (layer "F.Cu") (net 3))
 (segment (start 71.12 68.58) (end 78.74 68.58) (width 0.2) (layer "F.Cu") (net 3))
 (via (at 78.74 101.6) (size 0.6) (drill 0.3) (layers "F.Cu" "B.Cu") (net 3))
 (via (at 124.46 63.5) (size 0.6) (drill 0.3) (layers "F.Cu" "B.Cu") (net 3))
 (via (at 78.74 68.58) (size 0.6) (drill 0.3) (layers "F.Cu" "B.Cu") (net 3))
 (via (at 124.46 55.88) (size 0.6) (drill 0.3) (layers "F.Cu" "B.Cu") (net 3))
 (via (at 78.74 55.88) (size 0.6) (drill 0.3) (layers "F.Cu" "B.Cu") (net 3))
 (via (at 78.74 86.36) (size 0.6) (drill 0.3) (layers "F.Cu" "B.Cu") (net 3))
 (segment (start 78.74 101.6) (end 78.74 111.76) (width 0.2) (layer "B.Cu") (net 3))
 (segment (start 78.74 68.58) (end 78.74 55.88) (width 0.2) (layer "B.Cu") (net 3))
 (segment (start 78.74 101.6) (end 78.74 86.36) (width 0.2) (layer "B.Cu") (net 3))
 (segment (start 78.74 111.76) (end 88.9 111.76) (width 0.2) (layer "B.Cu") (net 3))
 (segment (start 78.74 68.58) (end 78.74 86.36) (width 0.2) (layer "B.Cu") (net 3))
 (segment (start 124.46 63.5) (end 124.46 55.88) (width 0.2) (layer "B.Cu") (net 3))
 (segment (start 71.12 106.68) (end 88.9 106.68) (width 0.2) (layer "F.Cu") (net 12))
 (segment (start 71.12 109.22) (end 88.9 109.22) (width 0.2) (layer "F.Cu") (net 13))
 (segment (start 114.3 96.52) (end 115.57 96.52) (width 0.2) (layer "F.Cu") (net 9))
 (segment (start 115.57 96.52) (end 129.54 96.52) (width 0.2) (layer "F.Cu") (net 9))
 (segment (start 132.08 88.9) (end 129.54 88.9) (width 0.2) (layer "F.Cu") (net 9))
 (via (at 129.54 96.52) (size 0.6) (drill 0.3) (layers "F.Cu" "B.Cu") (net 9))
 (via (at 129.54 88.9) (size 0.6) (drill 0.3) (layers "F.Cu" "B.Cu") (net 9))
 (segment (start 129.54 88.9) (end 129.54 90.17) (width 0.2) (layer "B.Cu") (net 9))
 (segment (start 129.54 90.17) (end 129.54 96.52) (width 0.2) (layer "B.Cu") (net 9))
 (segment (start 132.08 78.74) (end 123.19 78.74) (width 0.2) (layer "F.Cu") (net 5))
 (segment (start 114.3 81.28) (end 123.19 81.28) (width 0.2) (layer "F.Cu") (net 5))
 (via (at 123.19 78.74) (size 0.6) (drill 0.3) (layers "F.Cu" "B.Cu") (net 5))
 (via (at 123.19 81.28) (size 0.6) (drill 0.3) (layers "F.Cu" "B.Cu") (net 5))
 (segment (start 123.19 80.01) (end 123.19 81.28) (width 0.2) (layer "B.Cu") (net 5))
 (segment (start 123.19 78.74) (end 123.19 80.01) (width 0.2) (layer "B.Cu") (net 5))
 (segment (start 132.08 81.28) (end 124.46 81.28) (width 0.2) (layer "F.Cu") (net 6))
 (segment (start 114.3 83.82) (end 124.46 83.82) (width 0.2) (layer "F.Cu") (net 6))
 (via (at 124.46 81.28) (size 0.6) (drill 0.3) (layers "F.Cu" "B.Cu") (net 6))
 (via (at 124.46 83.82) (size 0.6) (drill 0.3) (layers "F.Cu" "B.Cu") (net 6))
 (segment (start 124.46 81.28) (end 124.46 82.55) (width 0.2) (layer "B.Cu") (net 6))
 (segment (start 124.46 82.55) (end 124.46 83.82) (width 0.2) (layer "B.Cu") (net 6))
 (segment (start 114.3 91.44) (end 115.57 91.44) (width 0.2) (layer "F.Cu") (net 8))
 (segment (start 115.57 91.44) (end 127 91.44) (width 0.2) (layer "F.Cu") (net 8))
 (segment (start 132.08 86.36) (end 130.81 86.36) (width 0.2) (layer "F.Cu") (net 8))
 (segment (start 130.81 86.36) (end 127 86.36) (width 0.2) (layer "F.Cu") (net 8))
 (via (at 127 86.36) (size 0.6) (drill 0.3) (layers "F.Cu" "B.Cu") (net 8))
 (via (at 127 91.44) (size 0.6) (drill 0.3) (layers "F.Cu" "B.Cu") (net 8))
 (segment (start 127 91.44) (end 127 86.36) (width 0.2) (layer "B.Cu") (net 8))
 (segment (start 130.81 83.82) (end 129.54 83.82) (width 0.2) (layer "F.Cu") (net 7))
 (segment (start 129.54 83.82) (end 125.73 83.82) (width 0.2) (layer "F.Cu") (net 7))
 (segment (start 132.08 83.82) (end 130.81 83.82) (width 0.2) (layer "F.Cu") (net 7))
 (segment (start 114.3 88.9) (end 125.73 88.9) (width 0.2) (layer "F.Cu") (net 7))
 (via (at 125.73 83.82) (size 0.6) (drill 0.3) (layers "F.Cu" "B.Cu") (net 7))
 (via (at 125.73 88.9) (size 0.6) (drill 0.3) (layers "F.Cu" "B.Cu") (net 7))
 (segment (start 125.73 87.63) (end 125.73 83.82) (width 0.2) (layer "B.Cu") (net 7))
 (segment (start 125.73 88.9) (end 125.73 87.63) (width 0.2) (layer "B.Cu") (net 7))
 (segment (start 114.3 73.66) (end 118.11 73.66) (width 0.2) (layer "F.Cu") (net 16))
 (segment (start 132.08 68.58) (end 118.11 68.58) (width 0.2) (layer "F.Cu") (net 16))
 (via (at 118.11 68.58) (size 0.6) (drill 0.3) (layers "F.Cu" "B.Cu") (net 16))
 (via (at 118.11 73.66) (size 0.6) (drill 0.3) (layers "F.Cu" "B.Cu") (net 16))
 (segment (start 118.11 68.58) (end 118.11 73.66) (width 0.2) (layer "B.Cu") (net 16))
 (segment (start 132.08 73.66) (end 130.81 73.66) (width 0.2) (layer "F.Cu") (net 18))
 (segment (start 130.81 73.66) (end 121.92 73.66) (width 0.2) (layer "F.Cu") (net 18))
 (segment (start 114.3 78.74) (end 121.92 78.74) (width 0.2) (layer "F.Cu") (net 18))
 (via (at 121.92 73.66) (size 0.6) (drill 0.3) (layers "F.Cu" "B.Cu") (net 18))
 (via (at 121.92 78.74) (size 0.6) (drill 0.3) (layers "F.Cu" "B.Cu") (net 18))
 (segment (start 121.92 73.66) (end 121.92 78.74) (width 0.2) (layer "B.Cu") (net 18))
 (segment (start 132.08 71.12) (end 119.38 71.12) (width 0.2) (layer "F.Cu") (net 17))
 (segment (start 114.3 76.2) (end 115.57 76.2) (width 0.2) (layer "F.Cu") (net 17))
 (segment (start 115.57 76.2) (end 119.38 76.2) (width 0.2) (layer "F.Cu") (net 17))
 (via (at 119.38 71.12) (size 0.6) (drill 0.3) (layers "F.Cu" "B.Cu") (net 17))
 (via (at 119.38 76.2) (size 0.6) (drill 0.3) (layers "F.Cu" "B.Cu") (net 17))
 (segment (start 119.38 71.12) (end 119.38 76.2) (width 0.2) (layer "B.Cu") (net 17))
 (segment (start 87.63 104.14) (end 81.28 104.14) (width 0.2) (layer "F.Cu") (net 11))
 (segment (start 88.9 104.14) (end 87.63 104.14) (width 0.2) (layer "F.Cu") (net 11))
 (segment (start 71.12 83.82) (end 81.28 83.82) (width 0.2) (layer "F.Cu") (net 11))
 (via (at 81.28 83.82) (size 0.6) (drill 0.3) (layers "F.Cu" "B.Cu") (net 11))
 (via (at 81.28 104.14) (size 0.6) (drill 0.3) (layers "F.Cu" "B.Cu") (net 11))
 (segment (start 81.28 104.14) (end 81.28 83.82) (width 0.2) (layer "B.Cu") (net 11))
 (segment (start 83.82 101.6) (end 82.55 101.6) (width 0.2) (layer "F.Cu") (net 10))
 (segment (start 71.12 81.28) (end 82.55 81.28) (width 0.2) (layer "F.Cu") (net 10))
 (segment (start 88.9 101.6) (end 87.63 101.6) (width 0.2) (layer "F.Cu") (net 10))
 (segment (start 87.63 101.6) (end 83.82 101.6) (width 0.2) (layer "F.Cu") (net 10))
 (via (at 82.55 81.28) (size 0.6) (drill 0.3) (layers "F.Cu" "B.Cu") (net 10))
 (via (at 82.55 101.6) (size 0.6) (drill 0.3) (layers "F.Cu" "B.Cu") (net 10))
 (segment (start 82.55 101.6) (end 82.55 81.28) (width 0.2) (layer "B.Cu") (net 10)))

